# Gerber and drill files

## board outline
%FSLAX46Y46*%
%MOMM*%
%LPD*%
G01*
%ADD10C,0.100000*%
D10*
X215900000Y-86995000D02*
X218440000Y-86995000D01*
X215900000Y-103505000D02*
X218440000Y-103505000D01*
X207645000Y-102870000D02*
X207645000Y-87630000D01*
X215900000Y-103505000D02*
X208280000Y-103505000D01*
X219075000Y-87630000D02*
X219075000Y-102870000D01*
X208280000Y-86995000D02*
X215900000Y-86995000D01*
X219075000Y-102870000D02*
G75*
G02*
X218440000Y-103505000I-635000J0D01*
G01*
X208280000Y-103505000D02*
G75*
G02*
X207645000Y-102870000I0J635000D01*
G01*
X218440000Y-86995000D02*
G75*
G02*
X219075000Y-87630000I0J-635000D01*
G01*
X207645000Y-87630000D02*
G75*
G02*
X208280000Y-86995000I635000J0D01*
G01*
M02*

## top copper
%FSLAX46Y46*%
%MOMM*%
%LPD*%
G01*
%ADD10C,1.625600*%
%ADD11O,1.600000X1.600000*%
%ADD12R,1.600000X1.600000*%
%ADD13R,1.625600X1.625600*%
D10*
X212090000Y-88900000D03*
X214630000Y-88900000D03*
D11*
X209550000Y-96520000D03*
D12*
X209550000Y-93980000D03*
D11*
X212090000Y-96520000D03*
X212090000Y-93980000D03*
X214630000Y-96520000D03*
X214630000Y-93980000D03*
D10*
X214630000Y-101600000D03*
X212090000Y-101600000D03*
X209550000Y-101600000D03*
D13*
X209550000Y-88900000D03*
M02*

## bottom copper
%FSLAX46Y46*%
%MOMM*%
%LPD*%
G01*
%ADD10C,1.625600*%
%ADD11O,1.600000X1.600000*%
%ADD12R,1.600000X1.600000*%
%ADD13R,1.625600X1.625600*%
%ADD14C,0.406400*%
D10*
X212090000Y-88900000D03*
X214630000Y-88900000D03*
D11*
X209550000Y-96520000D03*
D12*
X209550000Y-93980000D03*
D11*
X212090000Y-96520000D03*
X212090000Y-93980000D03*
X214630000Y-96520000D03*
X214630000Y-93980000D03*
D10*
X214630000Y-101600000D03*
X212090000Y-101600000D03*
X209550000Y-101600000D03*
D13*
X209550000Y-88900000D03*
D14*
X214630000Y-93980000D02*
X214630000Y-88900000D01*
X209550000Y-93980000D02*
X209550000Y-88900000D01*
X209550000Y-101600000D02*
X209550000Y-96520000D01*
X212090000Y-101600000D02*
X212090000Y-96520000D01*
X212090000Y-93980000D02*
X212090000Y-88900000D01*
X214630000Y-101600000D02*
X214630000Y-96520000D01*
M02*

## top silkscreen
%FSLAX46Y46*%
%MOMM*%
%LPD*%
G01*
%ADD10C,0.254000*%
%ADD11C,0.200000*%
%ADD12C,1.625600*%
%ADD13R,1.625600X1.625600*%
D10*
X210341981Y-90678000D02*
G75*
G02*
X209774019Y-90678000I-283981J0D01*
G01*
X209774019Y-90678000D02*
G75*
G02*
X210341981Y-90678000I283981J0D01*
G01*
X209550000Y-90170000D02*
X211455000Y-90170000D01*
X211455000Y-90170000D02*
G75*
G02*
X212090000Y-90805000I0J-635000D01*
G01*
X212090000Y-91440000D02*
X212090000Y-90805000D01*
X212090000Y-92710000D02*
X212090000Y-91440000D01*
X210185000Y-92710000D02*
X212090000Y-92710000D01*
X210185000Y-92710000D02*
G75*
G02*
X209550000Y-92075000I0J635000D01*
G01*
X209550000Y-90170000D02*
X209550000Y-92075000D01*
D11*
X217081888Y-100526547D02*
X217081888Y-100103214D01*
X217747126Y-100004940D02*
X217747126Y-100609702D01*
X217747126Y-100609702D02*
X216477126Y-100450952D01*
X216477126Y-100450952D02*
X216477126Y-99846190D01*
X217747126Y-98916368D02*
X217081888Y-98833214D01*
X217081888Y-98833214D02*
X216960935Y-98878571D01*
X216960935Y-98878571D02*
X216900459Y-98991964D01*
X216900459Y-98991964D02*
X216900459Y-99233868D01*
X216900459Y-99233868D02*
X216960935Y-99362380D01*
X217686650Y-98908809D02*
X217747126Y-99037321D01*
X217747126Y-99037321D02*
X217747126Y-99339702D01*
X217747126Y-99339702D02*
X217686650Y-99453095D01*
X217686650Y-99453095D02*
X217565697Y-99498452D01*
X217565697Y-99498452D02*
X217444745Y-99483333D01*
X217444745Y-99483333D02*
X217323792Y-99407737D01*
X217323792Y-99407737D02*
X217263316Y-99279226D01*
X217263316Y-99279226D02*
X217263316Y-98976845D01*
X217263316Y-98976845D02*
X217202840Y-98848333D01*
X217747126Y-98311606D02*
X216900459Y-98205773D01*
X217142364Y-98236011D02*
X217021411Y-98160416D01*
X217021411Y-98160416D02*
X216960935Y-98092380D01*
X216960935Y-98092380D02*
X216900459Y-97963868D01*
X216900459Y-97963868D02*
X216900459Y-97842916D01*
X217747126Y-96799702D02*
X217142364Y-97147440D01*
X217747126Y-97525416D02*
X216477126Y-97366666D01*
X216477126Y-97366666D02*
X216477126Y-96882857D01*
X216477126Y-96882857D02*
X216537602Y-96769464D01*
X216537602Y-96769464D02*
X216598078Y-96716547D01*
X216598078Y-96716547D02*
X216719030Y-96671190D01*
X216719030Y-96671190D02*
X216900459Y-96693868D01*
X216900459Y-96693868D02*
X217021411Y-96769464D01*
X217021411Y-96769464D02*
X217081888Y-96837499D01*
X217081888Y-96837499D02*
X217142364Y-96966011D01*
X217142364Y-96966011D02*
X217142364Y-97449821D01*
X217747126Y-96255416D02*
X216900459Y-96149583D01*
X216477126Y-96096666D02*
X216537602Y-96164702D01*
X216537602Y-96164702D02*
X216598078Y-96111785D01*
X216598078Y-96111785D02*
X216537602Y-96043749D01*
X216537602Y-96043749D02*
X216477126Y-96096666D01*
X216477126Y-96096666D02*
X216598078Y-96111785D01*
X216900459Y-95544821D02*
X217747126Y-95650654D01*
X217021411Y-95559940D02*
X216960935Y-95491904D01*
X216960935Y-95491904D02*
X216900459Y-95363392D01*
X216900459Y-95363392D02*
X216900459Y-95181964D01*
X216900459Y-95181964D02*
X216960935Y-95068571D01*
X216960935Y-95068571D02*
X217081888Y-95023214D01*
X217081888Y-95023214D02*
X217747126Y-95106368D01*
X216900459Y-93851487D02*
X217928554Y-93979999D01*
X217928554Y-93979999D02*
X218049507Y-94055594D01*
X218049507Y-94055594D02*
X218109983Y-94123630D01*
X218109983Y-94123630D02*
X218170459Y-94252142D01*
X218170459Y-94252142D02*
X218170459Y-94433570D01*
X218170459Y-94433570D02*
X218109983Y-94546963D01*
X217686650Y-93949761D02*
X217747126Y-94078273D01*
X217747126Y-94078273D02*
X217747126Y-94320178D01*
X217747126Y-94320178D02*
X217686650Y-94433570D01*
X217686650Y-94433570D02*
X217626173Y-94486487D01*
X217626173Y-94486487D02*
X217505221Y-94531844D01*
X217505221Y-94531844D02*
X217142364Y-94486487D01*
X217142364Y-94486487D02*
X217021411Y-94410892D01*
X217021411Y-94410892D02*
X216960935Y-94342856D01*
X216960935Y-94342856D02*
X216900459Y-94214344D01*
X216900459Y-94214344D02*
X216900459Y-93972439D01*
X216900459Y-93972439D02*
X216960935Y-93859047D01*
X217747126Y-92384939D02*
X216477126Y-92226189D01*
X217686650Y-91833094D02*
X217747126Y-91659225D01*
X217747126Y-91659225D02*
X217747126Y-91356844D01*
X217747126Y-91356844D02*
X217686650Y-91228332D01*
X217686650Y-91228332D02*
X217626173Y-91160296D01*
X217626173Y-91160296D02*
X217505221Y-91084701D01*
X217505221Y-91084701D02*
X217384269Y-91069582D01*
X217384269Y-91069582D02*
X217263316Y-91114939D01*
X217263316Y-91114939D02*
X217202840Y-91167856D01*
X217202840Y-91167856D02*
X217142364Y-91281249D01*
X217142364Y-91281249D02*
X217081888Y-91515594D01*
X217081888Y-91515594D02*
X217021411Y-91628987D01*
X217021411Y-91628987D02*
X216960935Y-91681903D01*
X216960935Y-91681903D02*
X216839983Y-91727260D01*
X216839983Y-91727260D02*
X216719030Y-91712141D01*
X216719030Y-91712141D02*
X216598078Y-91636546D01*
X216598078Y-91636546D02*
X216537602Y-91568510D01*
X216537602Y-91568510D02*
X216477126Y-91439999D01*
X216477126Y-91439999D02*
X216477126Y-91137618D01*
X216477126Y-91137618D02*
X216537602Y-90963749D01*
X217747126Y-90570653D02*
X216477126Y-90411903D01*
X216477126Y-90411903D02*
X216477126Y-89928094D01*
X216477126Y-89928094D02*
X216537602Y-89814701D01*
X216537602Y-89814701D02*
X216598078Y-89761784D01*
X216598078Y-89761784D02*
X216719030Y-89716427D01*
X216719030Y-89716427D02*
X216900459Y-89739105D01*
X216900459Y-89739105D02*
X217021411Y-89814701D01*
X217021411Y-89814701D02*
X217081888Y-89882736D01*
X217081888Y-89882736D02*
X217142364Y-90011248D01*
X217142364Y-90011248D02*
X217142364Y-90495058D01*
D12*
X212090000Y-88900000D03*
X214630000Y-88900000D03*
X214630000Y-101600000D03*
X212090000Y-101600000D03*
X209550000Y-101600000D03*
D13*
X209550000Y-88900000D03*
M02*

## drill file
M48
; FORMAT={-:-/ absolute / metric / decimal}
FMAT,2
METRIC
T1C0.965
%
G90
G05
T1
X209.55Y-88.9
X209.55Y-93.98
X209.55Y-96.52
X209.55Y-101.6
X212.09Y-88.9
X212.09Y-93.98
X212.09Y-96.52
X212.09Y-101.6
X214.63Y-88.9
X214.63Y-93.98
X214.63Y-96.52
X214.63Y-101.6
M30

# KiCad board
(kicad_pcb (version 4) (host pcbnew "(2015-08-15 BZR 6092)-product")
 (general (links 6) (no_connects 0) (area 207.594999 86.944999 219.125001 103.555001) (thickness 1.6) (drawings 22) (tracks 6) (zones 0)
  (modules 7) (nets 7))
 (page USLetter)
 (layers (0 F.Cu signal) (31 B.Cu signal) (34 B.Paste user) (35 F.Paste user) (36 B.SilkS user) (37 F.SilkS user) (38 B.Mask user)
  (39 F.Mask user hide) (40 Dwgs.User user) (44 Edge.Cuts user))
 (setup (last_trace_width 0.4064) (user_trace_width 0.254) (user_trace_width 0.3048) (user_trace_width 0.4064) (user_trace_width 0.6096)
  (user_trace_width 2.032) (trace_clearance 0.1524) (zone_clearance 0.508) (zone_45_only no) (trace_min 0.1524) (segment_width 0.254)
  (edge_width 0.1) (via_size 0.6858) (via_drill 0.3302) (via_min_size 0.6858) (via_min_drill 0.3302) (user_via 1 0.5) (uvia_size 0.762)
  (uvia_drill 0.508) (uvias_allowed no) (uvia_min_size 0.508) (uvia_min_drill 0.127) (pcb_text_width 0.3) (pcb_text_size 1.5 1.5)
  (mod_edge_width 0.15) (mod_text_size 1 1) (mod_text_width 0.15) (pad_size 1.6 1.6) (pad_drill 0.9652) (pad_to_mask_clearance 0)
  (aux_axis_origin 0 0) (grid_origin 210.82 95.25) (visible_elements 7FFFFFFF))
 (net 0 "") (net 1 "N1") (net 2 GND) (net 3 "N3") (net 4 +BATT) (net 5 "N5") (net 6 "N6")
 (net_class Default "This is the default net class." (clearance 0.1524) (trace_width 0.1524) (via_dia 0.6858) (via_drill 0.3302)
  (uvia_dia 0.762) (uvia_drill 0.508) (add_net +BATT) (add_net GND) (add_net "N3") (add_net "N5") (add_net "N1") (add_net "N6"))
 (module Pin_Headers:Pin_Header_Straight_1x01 (layer F.Cu) (at 212.09 88.9)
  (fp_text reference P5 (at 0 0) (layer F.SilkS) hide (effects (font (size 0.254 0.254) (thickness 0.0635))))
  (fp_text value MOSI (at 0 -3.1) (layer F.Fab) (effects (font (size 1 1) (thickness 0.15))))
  (pad 1 thru_hole circle (at 0 0) (size 1.6256 1.6256) (drill 0.9652) (layers *.Cu F.SilkS F.Mask) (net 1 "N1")))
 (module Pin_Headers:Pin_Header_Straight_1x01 (layer F.Cu) (at 214.63 88.9)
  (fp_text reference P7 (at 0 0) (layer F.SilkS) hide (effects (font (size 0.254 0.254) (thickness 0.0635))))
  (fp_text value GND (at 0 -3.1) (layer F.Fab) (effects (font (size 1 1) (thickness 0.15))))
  (pad 1 thru_hole circle (at 0 0) (size 1.6256 1.6256) (drill 0.9652) (layers *.Cu F.SilkS F.Mask) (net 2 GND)))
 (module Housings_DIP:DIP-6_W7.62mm (layer F.Cu) (at 209.55 96.52 90)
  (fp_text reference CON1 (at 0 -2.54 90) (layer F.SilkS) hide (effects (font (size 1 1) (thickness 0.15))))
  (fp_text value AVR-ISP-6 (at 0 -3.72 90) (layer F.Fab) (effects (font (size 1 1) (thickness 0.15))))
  (pad 1 thru_hole oval (at 0 0 90) (size 1.6 1.6) (drill 0.9652) (layers *.Cu B.SilkS B.Mask) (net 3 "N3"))
  (pad 2 thru_hole rect (at 2.54 0 90) (size 1.6 1.6) (drill 0.9652) (layers *.Cu B.SilkS B.Mask) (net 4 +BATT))
  (pad 3 thru_hole oval (at 0 2.54 90) (size 1.6 1.6) (drill 0.9652) (layers *.Cu B.SilkS B.Mask) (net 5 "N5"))
  (pad 4 thru_hole oval (at 2.54 2.54 90) (size 1.6 1.6) (drill 0.9652) (layers *.Cu B.SilkS B.Mask) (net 1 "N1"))
  (pad 5 thru_hole oval (at 0 5.08 90) (size 1.6 1.6) (drill 0.9652) (layers *.Cu B.SilkS B.Mask) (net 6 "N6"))
  (pad 6 thru_hole oval (at 2.54 5.08 90) (size 1.6 1.6) (drill 0.9652) (layers *.Cu B.SilkS B.Mask) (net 2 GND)))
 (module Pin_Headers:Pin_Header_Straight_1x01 (layer F.Cu) (at 214.63 101.6)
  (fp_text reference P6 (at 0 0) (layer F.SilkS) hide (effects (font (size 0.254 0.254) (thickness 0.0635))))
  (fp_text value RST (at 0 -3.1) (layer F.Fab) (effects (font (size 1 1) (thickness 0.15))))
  (pad 1 thru_hole circle (at 0 0) (size 1.6256 1.6256) (drill 0.9652) (layers *.Cu F.SilkS F.Mask) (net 6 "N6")))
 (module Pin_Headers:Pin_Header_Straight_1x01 (layer F.Cu) (at 212.09 101.6)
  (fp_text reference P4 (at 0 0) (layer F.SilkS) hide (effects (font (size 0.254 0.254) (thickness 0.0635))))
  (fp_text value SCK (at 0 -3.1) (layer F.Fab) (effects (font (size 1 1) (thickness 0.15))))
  (pad 1 thru_hole circle (at 0 0) (size 1.6256 1.6256) (drill 0.9652) (layers *.Cu F.SilkS F.Mask) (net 5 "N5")))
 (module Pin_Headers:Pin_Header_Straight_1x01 (layer F.Cu) (at 209.55 101.6)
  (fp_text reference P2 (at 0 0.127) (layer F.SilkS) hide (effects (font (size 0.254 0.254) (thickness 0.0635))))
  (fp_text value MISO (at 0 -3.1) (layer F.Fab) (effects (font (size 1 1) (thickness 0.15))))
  (pad 1 thru_hole circle (at 0 0) (size 1.6256 1.6256) (drill 0.9652) (layers *.Cu F.SilkS F.Mask) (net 3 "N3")))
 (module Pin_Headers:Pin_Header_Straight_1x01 (layer F.Cu) (at 209.55 88.9)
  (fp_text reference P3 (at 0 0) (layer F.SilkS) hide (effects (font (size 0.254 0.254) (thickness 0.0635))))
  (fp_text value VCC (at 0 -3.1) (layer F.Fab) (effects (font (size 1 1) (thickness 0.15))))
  (pad 1 thru_hole rect (at 0 0) (size 1.6256 1.6256) (drill 0.9652) (layers *.Cu F.SilkS F.Mask) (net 4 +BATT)))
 (gr_line (start 215.9 86.995) (end 218.44 86.995) (angle 90) (layer Edge.Cuts) (width 0.1))
 (gr_line (start 215.9 103.505) (end 218.44 103.505) (angle 90) (layer Edge.Cuts) (width 0.1))
 (gr_line (start 207.645 102.87) (end 207.645 87.63) (angle 90) (layer Edge.Cuts) (width 0.1))
 (gr_line (start 215.9 103.505) (end 208.28 103.505) (angle 90) (layer Edge.Cuts) (width 0.1))
 (gr_line (start 219.075 87.63) (end 219.075 102.87) (angle 90) (layer Edge.Cuts) (width 0.1))
 (gr_line (start 208.28 86.995) (end 215.9 86.995) (angle 90) (layer Edge.Cuts) (width 0.1))
 (gr_circle (center 210.058 90.678) (end 209.804 90.551) (layer F.SilkS) (width 0.254))
 (gr_line (start 209.55 90.17) (end 211.455 90.17) (angle 90) (layer F.SilkS) (width 0.254))
 (gr_arc (start 211.455 90.805) (end 211.455 90.17) (angle 90) (layer F.SilkS) (width 0.254))
 (gr_line (start 212.09 91.44) (end 212.09 90.805) (angle 90) (layer F.SilkS) (width 0.254))
 (gr_line (start 212.09 92.71) (end 212.09 91.44) (angle 90) (layer F.SilkS) (width 0.254))
 (gr_line (start 210.185 92.71) (end 212.09 92.71) (angle 90) (layer F.SilkS) (width 0.254))
 (gr_arc (start 210.185 92.075) (end 210.185 92.71) (angle 90) (layer F.SilkS) (width 0.254))
 (gr_line (start 209.55 90.17) (end 209.55 92.075) (angle 90) (layer F.SilkS) (width 0.254))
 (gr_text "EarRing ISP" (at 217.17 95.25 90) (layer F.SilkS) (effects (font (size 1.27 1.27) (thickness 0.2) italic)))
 (gr_arc (start 218.44 102.87) (end 219.075 102.87) (angle 90) (layer Edge.Cuts) (width 0.1))
 (gr_arc (start 208.28 102.87) (end 208.28 103.505) (angle 90) (layer Edge.Cuts) (width 0.1))
 (gr_arc (start 218.44 87.63) (end 218.44 86.995) (angle 90) (layer Edge.Cuts) (width 0.1))
 (gr_arc (start 208.28 87.63) (end 207.645 87.63) (angle 90) (layer Edge.Cuts) (width 0.1))
 (segment (start 214.63 93.98) (end 214.63 88.9) (width 0.4064) (layer B.Cu) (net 2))
 (segment (start 209.55 93.98) (end 209.55 88.9) (width 0.4064) (layer B.Cu) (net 4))
 (segment (start 209.55 101.6) (end 209.55 96.52) (width 0.4064) (layer B.Cu) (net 3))
 (segment (start 212.09 101.6) (end 212.09 96.52) (width 0.4064) (layer B.Cu) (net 5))
 (segment (start 212.09 93.98) (end 212.09 88.9) (width 0.4064) (layer B.Cu) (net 1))
 (segment (start 214.63 101.6) (end 214.63 96.52) (width 0.4064) (layer B.Cu) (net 6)))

